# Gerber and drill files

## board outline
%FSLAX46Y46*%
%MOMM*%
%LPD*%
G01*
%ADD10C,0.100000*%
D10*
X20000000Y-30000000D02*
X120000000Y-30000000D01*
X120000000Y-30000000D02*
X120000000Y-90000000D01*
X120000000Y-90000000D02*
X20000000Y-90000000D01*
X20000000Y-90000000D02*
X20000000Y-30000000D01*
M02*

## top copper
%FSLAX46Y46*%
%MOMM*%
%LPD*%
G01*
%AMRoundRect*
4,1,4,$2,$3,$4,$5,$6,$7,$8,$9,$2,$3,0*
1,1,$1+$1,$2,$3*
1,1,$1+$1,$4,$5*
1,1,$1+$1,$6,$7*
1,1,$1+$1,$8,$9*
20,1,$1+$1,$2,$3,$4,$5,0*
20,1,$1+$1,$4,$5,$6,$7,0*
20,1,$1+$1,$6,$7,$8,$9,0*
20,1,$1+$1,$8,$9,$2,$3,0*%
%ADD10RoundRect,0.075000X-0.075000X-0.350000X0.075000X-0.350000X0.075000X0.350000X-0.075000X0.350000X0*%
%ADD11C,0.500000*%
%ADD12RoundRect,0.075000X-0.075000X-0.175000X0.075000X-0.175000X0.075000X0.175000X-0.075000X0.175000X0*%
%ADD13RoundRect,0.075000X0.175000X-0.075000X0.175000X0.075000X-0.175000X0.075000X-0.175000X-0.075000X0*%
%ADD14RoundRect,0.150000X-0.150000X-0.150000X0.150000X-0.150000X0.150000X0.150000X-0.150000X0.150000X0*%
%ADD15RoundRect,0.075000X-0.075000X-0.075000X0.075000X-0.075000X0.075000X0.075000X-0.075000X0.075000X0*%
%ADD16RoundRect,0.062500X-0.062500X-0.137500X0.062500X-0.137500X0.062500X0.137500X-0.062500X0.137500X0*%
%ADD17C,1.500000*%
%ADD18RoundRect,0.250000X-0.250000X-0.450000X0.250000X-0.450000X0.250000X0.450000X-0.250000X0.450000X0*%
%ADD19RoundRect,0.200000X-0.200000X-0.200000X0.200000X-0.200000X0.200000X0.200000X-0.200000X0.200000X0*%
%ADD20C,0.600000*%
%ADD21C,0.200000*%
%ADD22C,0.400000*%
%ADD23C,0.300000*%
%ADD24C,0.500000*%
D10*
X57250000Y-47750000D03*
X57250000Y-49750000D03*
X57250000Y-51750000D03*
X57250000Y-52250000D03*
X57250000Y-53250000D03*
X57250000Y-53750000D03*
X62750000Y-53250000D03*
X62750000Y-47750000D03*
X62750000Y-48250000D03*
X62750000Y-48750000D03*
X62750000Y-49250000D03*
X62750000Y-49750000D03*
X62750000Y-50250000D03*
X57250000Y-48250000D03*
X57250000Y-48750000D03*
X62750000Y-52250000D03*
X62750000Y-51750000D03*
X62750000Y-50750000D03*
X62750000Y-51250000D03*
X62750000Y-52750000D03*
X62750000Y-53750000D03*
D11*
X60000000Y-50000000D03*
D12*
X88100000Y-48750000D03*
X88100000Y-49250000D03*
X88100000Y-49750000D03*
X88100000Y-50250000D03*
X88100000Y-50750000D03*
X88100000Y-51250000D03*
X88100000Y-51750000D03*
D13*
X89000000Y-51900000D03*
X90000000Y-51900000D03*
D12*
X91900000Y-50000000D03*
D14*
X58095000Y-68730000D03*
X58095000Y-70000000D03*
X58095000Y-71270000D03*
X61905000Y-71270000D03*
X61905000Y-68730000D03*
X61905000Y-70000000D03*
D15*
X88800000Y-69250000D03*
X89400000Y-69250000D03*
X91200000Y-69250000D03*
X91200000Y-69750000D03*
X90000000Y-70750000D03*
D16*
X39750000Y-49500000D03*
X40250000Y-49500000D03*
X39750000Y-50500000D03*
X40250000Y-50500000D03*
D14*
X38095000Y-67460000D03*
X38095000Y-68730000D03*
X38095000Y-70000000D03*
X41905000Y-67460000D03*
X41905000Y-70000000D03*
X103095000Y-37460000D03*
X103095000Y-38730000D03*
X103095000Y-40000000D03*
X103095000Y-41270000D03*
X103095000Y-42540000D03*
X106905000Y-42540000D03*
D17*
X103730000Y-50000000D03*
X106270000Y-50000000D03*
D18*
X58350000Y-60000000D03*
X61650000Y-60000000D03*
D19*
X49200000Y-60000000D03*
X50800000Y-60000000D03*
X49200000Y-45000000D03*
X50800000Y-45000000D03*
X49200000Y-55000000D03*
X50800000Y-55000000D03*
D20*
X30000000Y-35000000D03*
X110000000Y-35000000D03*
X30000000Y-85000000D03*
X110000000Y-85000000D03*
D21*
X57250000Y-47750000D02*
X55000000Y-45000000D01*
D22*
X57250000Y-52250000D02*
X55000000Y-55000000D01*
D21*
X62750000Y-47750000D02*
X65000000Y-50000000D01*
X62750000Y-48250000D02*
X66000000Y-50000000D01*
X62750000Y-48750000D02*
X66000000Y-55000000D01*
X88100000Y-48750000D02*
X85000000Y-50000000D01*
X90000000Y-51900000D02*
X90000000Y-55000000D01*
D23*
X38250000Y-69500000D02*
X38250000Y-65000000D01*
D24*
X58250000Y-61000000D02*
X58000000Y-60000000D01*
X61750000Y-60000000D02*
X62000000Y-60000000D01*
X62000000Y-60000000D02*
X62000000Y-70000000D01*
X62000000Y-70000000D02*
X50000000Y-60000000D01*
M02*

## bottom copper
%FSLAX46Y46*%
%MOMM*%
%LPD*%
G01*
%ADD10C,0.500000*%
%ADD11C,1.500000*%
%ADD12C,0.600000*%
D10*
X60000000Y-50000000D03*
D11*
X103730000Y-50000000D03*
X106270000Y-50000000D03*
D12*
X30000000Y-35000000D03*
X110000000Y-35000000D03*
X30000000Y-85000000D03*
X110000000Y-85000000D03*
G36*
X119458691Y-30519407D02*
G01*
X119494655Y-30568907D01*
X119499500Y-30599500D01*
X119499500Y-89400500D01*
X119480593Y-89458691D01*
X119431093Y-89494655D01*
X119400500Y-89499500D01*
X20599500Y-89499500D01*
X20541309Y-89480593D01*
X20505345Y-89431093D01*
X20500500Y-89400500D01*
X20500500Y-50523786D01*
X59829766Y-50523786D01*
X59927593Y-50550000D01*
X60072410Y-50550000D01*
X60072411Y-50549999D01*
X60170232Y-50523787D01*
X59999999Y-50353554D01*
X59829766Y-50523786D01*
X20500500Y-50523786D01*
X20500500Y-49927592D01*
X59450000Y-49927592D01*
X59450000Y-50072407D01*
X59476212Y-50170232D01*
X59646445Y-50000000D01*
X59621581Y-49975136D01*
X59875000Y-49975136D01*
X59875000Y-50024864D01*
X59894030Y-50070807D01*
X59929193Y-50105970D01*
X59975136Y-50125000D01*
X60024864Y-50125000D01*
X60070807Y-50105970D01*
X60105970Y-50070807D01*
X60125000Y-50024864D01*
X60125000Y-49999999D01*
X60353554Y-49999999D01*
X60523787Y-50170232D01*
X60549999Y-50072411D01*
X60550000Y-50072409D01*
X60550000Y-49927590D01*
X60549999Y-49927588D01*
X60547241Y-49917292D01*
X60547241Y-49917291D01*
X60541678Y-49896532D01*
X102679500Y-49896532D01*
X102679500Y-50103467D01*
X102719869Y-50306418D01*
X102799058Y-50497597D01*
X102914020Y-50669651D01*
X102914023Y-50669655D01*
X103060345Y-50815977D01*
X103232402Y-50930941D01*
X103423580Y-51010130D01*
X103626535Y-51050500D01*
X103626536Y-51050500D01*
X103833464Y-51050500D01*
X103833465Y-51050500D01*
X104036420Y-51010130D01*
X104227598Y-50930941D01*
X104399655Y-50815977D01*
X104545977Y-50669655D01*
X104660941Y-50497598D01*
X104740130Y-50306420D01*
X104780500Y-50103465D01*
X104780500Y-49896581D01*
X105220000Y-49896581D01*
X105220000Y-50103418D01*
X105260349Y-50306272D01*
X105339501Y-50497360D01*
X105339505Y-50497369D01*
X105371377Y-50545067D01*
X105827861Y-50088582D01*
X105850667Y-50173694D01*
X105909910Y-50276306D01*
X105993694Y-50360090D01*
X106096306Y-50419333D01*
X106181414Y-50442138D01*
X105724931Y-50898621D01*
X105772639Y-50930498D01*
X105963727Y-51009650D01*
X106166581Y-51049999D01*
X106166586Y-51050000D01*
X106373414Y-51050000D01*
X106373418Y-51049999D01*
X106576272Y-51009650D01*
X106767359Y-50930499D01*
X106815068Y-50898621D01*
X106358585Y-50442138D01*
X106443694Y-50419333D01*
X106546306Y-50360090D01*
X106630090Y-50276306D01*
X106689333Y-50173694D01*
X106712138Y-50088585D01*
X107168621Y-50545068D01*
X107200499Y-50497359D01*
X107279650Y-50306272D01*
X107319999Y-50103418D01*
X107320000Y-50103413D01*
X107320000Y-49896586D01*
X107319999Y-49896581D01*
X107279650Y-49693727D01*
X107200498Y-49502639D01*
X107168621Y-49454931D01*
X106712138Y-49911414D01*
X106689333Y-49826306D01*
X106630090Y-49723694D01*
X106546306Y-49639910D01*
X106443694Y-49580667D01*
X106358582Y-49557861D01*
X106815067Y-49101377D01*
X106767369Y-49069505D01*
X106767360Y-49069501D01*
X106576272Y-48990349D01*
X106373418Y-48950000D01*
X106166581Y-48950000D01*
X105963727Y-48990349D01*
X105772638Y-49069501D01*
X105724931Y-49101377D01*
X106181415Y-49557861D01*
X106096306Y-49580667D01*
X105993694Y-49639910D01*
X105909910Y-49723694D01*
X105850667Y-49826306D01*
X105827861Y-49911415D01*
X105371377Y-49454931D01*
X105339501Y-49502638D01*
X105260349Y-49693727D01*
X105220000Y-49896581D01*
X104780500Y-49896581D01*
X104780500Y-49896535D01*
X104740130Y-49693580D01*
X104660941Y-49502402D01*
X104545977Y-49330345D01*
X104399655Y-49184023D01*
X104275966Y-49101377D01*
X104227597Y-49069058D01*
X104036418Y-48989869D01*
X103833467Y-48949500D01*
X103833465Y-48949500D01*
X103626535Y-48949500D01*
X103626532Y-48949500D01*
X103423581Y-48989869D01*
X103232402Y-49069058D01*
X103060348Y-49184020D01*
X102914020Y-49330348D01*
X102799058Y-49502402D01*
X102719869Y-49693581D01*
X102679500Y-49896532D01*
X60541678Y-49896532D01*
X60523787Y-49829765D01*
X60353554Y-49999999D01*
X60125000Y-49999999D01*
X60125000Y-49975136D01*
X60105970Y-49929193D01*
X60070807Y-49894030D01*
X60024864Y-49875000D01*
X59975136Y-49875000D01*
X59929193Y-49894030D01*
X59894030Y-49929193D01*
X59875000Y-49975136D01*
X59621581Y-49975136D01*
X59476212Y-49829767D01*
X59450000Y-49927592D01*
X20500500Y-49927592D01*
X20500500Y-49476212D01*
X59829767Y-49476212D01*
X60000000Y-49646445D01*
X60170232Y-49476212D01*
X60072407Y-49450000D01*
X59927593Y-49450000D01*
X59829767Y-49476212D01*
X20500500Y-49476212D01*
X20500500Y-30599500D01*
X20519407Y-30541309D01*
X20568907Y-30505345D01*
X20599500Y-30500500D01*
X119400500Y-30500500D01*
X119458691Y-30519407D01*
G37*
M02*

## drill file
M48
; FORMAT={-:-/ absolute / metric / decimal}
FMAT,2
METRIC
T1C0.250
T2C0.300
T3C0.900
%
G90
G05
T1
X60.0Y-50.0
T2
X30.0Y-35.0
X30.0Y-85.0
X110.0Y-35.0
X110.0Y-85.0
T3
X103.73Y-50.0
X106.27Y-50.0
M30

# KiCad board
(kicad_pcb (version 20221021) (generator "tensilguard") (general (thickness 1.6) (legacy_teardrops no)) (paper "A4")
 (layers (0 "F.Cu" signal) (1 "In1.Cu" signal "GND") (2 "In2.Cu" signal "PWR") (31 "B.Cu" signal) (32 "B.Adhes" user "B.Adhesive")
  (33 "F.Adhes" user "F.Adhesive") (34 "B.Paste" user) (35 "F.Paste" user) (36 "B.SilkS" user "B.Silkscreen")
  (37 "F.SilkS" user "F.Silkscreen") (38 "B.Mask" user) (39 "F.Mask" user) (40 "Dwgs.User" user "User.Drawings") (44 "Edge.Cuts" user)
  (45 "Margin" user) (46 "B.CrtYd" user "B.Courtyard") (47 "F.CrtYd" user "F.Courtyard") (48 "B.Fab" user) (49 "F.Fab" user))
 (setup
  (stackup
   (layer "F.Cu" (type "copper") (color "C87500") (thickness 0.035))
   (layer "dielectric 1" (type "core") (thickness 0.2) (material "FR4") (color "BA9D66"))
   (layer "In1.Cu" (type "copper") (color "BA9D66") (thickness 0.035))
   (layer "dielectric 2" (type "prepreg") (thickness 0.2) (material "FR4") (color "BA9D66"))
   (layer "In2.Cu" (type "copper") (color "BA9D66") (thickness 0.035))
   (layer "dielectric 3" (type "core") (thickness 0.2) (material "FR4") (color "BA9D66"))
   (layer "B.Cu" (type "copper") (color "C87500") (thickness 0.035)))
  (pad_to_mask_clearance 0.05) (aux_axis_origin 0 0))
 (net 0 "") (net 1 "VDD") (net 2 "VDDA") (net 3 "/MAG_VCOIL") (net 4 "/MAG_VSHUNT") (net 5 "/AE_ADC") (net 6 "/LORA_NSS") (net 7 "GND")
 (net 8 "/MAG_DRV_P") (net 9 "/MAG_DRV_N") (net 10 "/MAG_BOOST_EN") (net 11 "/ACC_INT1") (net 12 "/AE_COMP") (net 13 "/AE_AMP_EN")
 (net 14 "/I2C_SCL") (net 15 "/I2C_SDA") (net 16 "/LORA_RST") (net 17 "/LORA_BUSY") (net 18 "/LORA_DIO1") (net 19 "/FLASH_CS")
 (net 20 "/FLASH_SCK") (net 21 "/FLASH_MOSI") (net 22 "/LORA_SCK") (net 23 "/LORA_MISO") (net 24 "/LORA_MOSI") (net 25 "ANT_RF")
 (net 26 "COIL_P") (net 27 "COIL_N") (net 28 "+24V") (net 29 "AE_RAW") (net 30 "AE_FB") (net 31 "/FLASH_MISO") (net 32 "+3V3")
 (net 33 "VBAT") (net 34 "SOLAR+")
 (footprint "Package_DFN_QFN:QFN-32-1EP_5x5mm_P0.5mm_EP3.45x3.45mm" (layer "F.Cu") (at 60 50)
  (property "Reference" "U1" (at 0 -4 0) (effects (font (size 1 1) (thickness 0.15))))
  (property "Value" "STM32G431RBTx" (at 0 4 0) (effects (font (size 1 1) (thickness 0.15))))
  (pad "1" smd roundrect (at -2.75 -2.25 0) (size 0.3 0.85) (layers "F.Cu" "F.Paste" "F.Mask") (roundrect_rratio 0.25) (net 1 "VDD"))
  (pad "5" smd roundrect (at -2.75 -0.25 0) (size 0.3 0.85) (layers "F.Cu" "F.Paste" "F.Mask") (roundrect_rratio 0.25) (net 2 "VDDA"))
  (pad "8" smd roundrect (at -2.75 1.75 0) (size 0.3 0.85) (layers "F.Cu" "F.Paste" "F.Mask") (roundrect_rratio 0.25) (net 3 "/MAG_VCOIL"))
  (pad "9" smd roundrect (at -2.75 2.25 0) (size 0.3 0.85) (layers "F.Cu" "F.Paste" "F.Mask") (roundrect_rratio 0.25) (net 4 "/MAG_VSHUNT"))
  (pad "11" smd roundrect (at -2.75 3.25 0) (size 0.3 0.85) (layers "F.Cu" "F.Paste" "F.Mask") (roundrect_rratio 0.25) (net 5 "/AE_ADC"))
  (pad "12" smd roundrect (at -2.75 3.75 0) (size 0.3 0.85) (layers "F.Cu" "F.Paste" "F.Mask") (roundrect_rratio 0.25) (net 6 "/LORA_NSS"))
  (pad "17" smd roundrect (at 2.75 3.25 0) (size 0.3 0.85) (layers "F.Cu" "F.Paste" "F.Mask") (roundrect_rratio 0.25) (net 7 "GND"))
  (pad "23" smd roundrect (at 2.75 -2.25 0) (size 0.3 0.85) (layers "F.Cu" "F.Paste" "F.Mask") (roundrect_rratio 0.25) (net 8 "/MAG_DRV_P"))
  (pad "24" smd roundrect (at 2.75 -1.75 0) (size 0.3 0.85) (layers "F.Cu" "F.Paste" "F.Mask") (roundrect_rratio 0.25) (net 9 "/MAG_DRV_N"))
  (pad "25" smd roundrect (at 2.75 -1.25 0) (size 0.3 0.85) (layers "F.Cu" "F.Paste" "F.Mask") (roundrect_rratio 0.25)
   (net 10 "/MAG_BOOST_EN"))
  (pad "26" smd roundrect (at 2.75 -0.75 0) (size 0.3 0.85) (layers "F.Cu" "F.Paste" "F.Mask") (roundrect_rratio 0.25) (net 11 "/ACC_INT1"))
  (pad "27" smd roundrect (at 2.75 -0.25 0) (size 0.3 0.85) (layers "F.Cu" "F.Paste" "F.Mask") (roundrect_rratio 0.25) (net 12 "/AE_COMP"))
  (pad "28" smd roundrect (at 2.75 0.25 0) (size 0.3 0.85) (layers "F.Cu" "F.Paste" "F.Mask") (roundrect_rratio 0.25) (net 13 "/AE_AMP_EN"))
  (pad "42" smd roundrect (at -2.75 -1.75 0) (size 0.3 0.85) (layers "F.Cu" "F.Paste" "F.Mask") (roundrect_rratio 0.25) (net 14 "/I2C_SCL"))
  (pad "43" smd roundrect (at -2.75 -1.25 0) (size 0.3 0.85) (layers "F.Cu" "F.Paste" "F.Mask") (roundrect_rratio 0.25) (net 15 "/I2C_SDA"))
  (pad "21" smd roundrect (at 2.75 2.25 0) (size 0.3 0.85) (layers "F.Cu" "F.Paste" "F.Mask") (roundrect_rratio 0.25) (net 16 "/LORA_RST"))
  (pad "22" smd roundrect (at 2.75 1.75 0) (size 0.3 0.85) (layers "F.Cu" "F.Paste" "F.Mask") (roundrect_rratio 0.25) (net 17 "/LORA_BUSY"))
  (pad "33" smd roundrect (at 2.75 0.75 0) (size 0.3 0.85) (layers "F.Cu" "F.Paste" "F.Mask") (roundrect_rratio 0.25) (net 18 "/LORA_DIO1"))
  (pad "34" smd roundrect (at 2.75 1.25 0) (size 0.3 0.85) (layers "F.Cu" "F.Paste" "F.Mask") (roundrect_rratio 0.25) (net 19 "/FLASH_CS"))
  (pad "35" smd roundrect (at 2.75 2.75 0) (size 0.3 0.85) (layers "F.Cu" "F.Paste" "F.Mask") (roundrect_rratio 0.25) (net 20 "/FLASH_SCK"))
  (pad "36" smd roundrect (at 2.75 3.75 0) (size 0.3 0.85) (layers "F.Cu" "F.Paste" "F.Mask") (roundrect_rratio 0.25) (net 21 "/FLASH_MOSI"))
  (pad "33_2" thru_hole circle (at 0 0 0) (size 0.5 0.5) (drill 0.25) (layers "*.Cu") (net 7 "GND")))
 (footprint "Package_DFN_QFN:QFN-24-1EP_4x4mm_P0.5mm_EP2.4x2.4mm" (layer "F.Cu") (at 90 50)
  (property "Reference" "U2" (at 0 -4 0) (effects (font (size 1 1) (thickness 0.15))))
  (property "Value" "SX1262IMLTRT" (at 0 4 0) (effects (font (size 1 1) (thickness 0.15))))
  (pad "1" smd roundrect (at -1.9 -1.25 0) (size 0.3 0.5) (layers "F.Cu" "F.Paste" "F.Mask") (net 7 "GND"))
  (pad "2" smd roundrect (at -1.9 -0.75 0) (size 0.3 0.5) (layers "F.Cu" "F.Paste" "F.Mask") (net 6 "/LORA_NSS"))
  (pad "3" smd roundrect (at -1.9 -0.25 0) (size 0.3 0.5) (layers "F.Cu" "F.Paste" "F.Mask") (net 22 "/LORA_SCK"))
  (pad "4" smd roundrect (at -1.9 0.25 0) (size 0.3 0.5) (layers "F.Cu" "F.Paste" "F.Mask") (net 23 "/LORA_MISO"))
  (pad "5" smd roundrect (at -1.9 0.75 0) (size 0.3 0.5) (layers "F.Cu" "F.Paste" "F.Mask") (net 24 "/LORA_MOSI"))
  (pad "6" smd roundrect (at -1.9 1.25 0) (size 0.3 0.5) (layers "F.Cu" "F.Paste" "F.Mask") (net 18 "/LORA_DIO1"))
  (pad "7" smd roundrect (at -1.9 1.75 0) (size 0.3 0.5) (layers "F.Cu" "F.Paste" "F.Mask") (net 17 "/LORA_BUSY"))
  (pad "9" smd roundrect (at -1 1.9 90) (size 0.3 0.5) (layers "F.Cu" "F.Paste" "F.Mask") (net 16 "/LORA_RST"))
  (pad "10" smd roundrect (at 0 1.9 90) (size 0.3 0.5) (layers "F.Cu" "F.Paste" "F.Mask") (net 1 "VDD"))
  (pad "21" smd roundrect (at 1.9 0 0) (size 0.3 0.5) (layers "F.Cu" "F.Paste" "F.Mask") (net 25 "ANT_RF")))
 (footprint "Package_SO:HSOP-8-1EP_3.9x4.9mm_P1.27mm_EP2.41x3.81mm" (layer "F.Cu") (at 60 70)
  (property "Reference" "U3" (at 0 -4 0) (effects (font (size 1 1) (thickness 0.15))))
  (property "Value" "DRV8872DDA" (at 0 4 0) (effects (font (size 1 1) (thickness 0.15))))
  (pad "1" smd roundrect (at -1.905 -1.27 0) (size 0.6 0.6) (layers "F.Cu" "F.Paste" "F.Mask") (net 8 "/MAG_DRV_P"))
  (pad "2" smd roundrect (at -1.905 0 0) (size 0.6 0.6) (layers "F.Cu" "F.Paste" "F.Mask") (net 9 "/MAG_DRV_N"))
  (pad "3" smd roundrect (at -1.905 1.27 0) (size 0.6 0.6) (layers "F.Cu" "F.Paste" "F.Mask") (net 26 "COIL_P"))
  (pad "4" smd roundrect (at 1.905 1.27 0) (size 0.6 0.6) (layers "F.Cu" "F.Paste" "F.Mask") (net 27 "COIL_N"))
  (pad "6" smd roundrect (at 1.905 -1.27 0) (size 0.6 0.6) (layers "F.Cu" "F.Paste" "F.Mask") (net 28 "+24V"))
  (pad "7" smd roundrect (at 1.905 0 0) (size 0.6 0.6) (layers "F.Cu" "F.Paste" "F.Mask") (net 7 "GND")))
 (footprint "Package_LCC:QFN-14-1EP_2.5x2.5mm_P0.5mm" (layer "F.Cu") (at 90 70)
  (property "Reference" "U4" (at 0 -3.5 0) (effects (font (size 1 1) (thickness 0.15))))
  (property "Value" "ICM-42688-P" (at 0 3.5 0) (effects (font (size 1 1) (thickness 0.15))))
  (pad "1" smd roundrect (at -1.2 -0.75 0) (size 0.3 0.3) (layers "F.Cu" "F.Paste" "F.Mask") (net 1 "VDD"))
  (pad "2" smd roundrect (at -0.6 -0.75 0) (size 0.3 0.3) (layers "F.Cu" "F.Paste" "F.Mask") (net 20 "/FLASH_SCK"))
  (pad "5" smd roundrect (at 1.2 -0.75 0) (size 0.3 0.3) (layers "F.Cu" "F.Paste" "F.Mask") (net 19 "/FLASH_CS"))
  (pad "6" smd roundrect (at 1.2 -0.25 0) (size 0.3 0.3) (layers "F.Cu" "F.Paste" "F.Mask") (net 11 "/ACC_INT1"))
  (pad "14" smd roundrect (at 0 0.75 0) (size 0.3 0.3) (layers "F.Cu" "F.Paste" "F.Mask") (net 7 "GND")))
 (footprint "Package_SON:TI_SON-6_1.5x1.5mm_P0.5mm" (layer "F.Cu") (at 40 50)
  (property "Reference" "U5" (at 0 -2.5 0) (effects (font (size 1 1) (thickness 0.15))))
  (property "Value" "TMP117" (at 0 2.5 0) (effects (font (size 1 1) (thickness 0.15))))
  (pad "1" smd roundrect (at -0.25 -0.5 0) (size 0.25 0.4) (layers "F.Cu" "F.Paste" "F.Mask") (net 1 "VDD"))
  (pad "2" smd roundrect (at 0.25 -0.5 0) (size 0.25 0.4) (layers "F.Cu" "F.Paste" "F.Mask") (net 7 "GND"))
  (pad "3" smd roundrect (at -0.25 0.5 0) (size 0.25 0.4) (layers "F.Cu" "F.Paste" "F.Mask") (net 15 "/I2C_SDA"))
  (pad "4" smd roundrect (at 0.25 0.5 0) (size 0.25 0.4) (layers "F.Cu" "F.Paste" "F.Mask") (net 14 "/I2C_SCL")))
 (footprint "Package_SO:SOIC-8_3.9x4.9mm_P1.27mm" (layer "F.Cu") (at 40 70)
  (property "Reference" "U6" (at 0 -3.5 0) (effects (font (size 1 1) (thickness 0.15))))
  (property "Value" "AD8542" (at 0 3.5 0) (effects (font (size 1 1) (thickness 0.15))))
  (pad "1" smd roundrect (at -1.905 -2.54 0) (size 0.6 0.6) (layers "F.Cu" "F.Paste" "F.Mask") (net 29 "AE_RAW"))
  (pad "2" smd roundrect (at -1.905 -1.27 0) (size 0.6 0.6) (layers "F.Cu" "F.Paste" "F.Mask") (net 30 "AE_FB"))
  (pad "3" smd roundrect (at -1.905 0 0) (size 0.6 0.6) (layers "F.Cu" "F.Paste" "F.Mask") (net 5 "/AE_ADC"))
  (pad "4" smd roundrect (at 1.905 -2.54 0) (size 0.6 0.6) (layers "F.Cu" "F.Paste" "F.Mask") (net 1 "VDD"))
  (pad "5" smd roundrect (at 1.905 0 0) (size 0.6 0.6) (layers "F.Cu" "F.Paste" "F.Mask") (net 7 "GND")))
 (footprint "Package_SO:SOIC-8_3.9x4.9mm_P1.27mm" (layer "F.Cu") (at 105 40)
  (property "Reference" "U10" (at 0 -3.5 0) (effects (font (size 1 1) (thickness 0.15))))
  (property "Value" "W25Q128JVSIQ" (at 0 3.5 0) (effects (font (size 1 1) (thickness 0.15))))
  (pad "1" smd roundrect (at -1.905 -2.54 0) (size 0.6 0.6) (layers "F.Cu" "F.Paste" "F.Mask") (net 1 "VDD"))
  (pad "2" smd roundrect (at -1.905 -1.27 0) (size 0.6 0.6) (layers "F.Cu" "F.Paste" "F.Mask") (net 19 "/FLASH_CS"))
  (pad "3" smd roundrect (at -1.905 0 0) (size 0.6 0.6) (layers "F.Cu" "F.Paste" "F.Mask") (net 20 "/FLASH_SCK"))
  (pad "4" smd roundrect (at -1.905 1.27 0) (size 0.6 0.6) (layers "F.Cu" "F.Paste" "F.Mask") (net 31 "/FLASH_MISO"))
  (pad "5" smd roundrect (at -1.905 2.54 0) (size 0.6 0.6) (layers "F.Cu" "F.Paste" "F.Mask") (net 21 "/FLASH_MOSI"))
  (pad "8" smd roundrect (at 1.905 2.54 0) (size 0.6 0.6) (layers "F.Cu" "F.Paste" "F.Mask") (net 7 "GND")))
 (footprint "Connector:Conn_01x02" (layer "F.Cu") (at 105 50)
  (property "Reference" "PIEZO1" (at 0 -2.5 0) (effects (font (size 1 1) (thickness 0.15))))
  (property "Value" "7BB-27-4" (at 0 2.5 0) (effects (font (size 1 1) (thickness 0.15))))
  (pad "1" thru_hole circle (at -1.27 0 0) (size 1.5 1.5) (drill 0.9) (layers "*.Cu" "*.Mask") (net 29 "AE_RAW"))
  (pad "2" thru_hole circle (at 1.27 0 0) (size 1.5 1.5) (drill 0.9) (layers "*.Cu" "*.Mask") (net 7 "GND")))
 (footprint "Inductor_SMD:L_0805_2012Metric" (layer "F.Cu") (at 60 60)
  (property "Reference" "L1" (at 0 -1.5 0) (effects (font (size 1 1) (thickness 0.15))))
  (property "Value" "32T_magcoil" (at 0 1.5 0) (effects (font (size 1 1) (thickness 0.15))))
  (pad "1" smd roundrect (at -1.65 0 0) (size 1 1.4) (layers "F.Cu" "F.Paste" "F.Mask") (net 26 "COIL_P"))
  (pad "2" smd roundrect (at 1.65 0 0) (size 1 1.4) (layers "F.Cu" "F.Paste" "F.Mask") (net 27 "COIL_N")))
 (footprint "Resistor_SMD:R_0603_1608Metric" (layer "F.Cu") (at 50 60)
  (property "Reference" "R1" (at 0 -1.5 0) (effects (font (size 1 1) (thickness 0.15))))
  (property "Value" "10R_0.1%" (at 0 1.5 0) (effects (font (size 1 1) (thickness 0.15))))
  (pad "1" smd roundrect (at -0.8 0 0) (size 0.8 0.8) (layers "F.Cu" "F.Paste" "F.Mask") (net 27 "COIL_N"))
  (pad "2" smd roundrect (at 0.8 0 0) (size 0.8 0.8) (layers "F.Cu" "F.Paste" "F.Mask") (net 7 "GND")))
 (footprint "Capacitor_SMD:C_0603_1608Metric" (layer "F.Cu") (at 50 45)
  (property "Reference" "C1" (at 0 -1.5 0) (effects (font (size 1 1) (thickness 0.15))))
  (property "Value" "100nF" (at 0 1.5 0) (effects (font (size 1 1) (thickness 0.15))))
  (pad "1" smd roundrect (at -0.8 0 0) (size 0.8 0.8) (layers "F.Cu" "F.Paste" "F.Mask") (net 1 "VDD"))
  (pad "2" smd roundrect (at 0.8 0 0) (size 0.8 0.8) (layers "F.Cu" "F.Paste" "F.Mask") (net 7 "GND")))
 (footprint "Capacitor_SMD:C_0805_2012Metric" (layer "F.Cu") (at 50 55)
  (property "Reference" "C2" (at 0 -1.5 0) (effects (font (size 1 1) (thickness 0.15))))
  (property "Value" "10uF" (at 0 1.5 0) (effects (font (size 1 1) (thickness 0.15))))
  (pad "1" smd roundrect (at -0.8 0 0) (size 0.8 0.8) (layers "F.Cu" "F.Paste" "F.Mask") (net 28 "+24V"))
  (pad "2" smd roundrect (at 0.8 0 0) (size 0.8 0.8) (layers "F.Cu" "F.Paste" "F.Mask") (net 7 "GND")))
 (gr_line (start 20 30) (end 120 30) (layer "Edge.Cuts") (stroke (width 0.1)))
 (gr_line (start 120 30) (end 120 90) (layer "Edge.Cuts") (stroke (width 0.1)))
 (gr_line (start 120 90) (end 20 90) (layer "Edge.Cuts") (stroke (width 0.1)))
 (gr_line (start 20 90) (end 20 30) (layer "Edge.Cuts") (stroke (width 0.1)))
 (segment (start 57.25 47.75) (end 55 45) (width 0.2) (layer "F.Cu") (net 1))
 (segment (start 57.25 52.25) (end 55 55) (width 0.4) (layer "F.Cu") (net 7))
 (segment (start 62.75 47.75) (end 65 50) (width 0.2) (layer "F.Cu") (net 8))
 (segment (start 62.75 48.25) (end 66 50) (width 0.2) (layer "F.Cu") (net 9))
 (segment (start 62.75 48.75) (end 66 55) (width 0.2) (layer "F.Cu") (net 10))
 (segment (start 88.1 48.75) (end 85 50) (width 0.2) (layer "F.Cu") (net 18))
 (segment (start 90 51.9) (end 90 55) (width 0.2) (layer "F.Cu") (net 1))
 (segment (start 38.25 69.5) (end 38.25 65) (width 0.3) (layer "F.Cu") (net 29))
 (segment (start 58.25 61) (end 58 60) (width 0.5) (layer "F.Cu") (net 26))
 (segment (start 61.75 60) (end 62 60) (width 0.5) (layer "F.Cu") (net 27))
 (segment (start 62 60) (end 62 70) (width 0.5) (layer "F.Cu") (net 27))
 (segment (start 62 70) (end 50 60) (width 0.5) (layer "F.Cu") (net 27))
 (via (at 30 35) (size 0.6) (drill 0.3) (layers "F.Cu" "B.Cu") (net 7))
 (via (at 110 35) (size 0.6) (drill 0.3) (layers "F.Cu" "B.Cu") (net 7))
 (via (at 30 85) (size 0.6) (drill 0.3) (layers "F.Cu" "B.Cu") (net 7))
 (via (at 110 85) (size 0.6) (drill 0.3) (layers "F.Cu" "B.Cu") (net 7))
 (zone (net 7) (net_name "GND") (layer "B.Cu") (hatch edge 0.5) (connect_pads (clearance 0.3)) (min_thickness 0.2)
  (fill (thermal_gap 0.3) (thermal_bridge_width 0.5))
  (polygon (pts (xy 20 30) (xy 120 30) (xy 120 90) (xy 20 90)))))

